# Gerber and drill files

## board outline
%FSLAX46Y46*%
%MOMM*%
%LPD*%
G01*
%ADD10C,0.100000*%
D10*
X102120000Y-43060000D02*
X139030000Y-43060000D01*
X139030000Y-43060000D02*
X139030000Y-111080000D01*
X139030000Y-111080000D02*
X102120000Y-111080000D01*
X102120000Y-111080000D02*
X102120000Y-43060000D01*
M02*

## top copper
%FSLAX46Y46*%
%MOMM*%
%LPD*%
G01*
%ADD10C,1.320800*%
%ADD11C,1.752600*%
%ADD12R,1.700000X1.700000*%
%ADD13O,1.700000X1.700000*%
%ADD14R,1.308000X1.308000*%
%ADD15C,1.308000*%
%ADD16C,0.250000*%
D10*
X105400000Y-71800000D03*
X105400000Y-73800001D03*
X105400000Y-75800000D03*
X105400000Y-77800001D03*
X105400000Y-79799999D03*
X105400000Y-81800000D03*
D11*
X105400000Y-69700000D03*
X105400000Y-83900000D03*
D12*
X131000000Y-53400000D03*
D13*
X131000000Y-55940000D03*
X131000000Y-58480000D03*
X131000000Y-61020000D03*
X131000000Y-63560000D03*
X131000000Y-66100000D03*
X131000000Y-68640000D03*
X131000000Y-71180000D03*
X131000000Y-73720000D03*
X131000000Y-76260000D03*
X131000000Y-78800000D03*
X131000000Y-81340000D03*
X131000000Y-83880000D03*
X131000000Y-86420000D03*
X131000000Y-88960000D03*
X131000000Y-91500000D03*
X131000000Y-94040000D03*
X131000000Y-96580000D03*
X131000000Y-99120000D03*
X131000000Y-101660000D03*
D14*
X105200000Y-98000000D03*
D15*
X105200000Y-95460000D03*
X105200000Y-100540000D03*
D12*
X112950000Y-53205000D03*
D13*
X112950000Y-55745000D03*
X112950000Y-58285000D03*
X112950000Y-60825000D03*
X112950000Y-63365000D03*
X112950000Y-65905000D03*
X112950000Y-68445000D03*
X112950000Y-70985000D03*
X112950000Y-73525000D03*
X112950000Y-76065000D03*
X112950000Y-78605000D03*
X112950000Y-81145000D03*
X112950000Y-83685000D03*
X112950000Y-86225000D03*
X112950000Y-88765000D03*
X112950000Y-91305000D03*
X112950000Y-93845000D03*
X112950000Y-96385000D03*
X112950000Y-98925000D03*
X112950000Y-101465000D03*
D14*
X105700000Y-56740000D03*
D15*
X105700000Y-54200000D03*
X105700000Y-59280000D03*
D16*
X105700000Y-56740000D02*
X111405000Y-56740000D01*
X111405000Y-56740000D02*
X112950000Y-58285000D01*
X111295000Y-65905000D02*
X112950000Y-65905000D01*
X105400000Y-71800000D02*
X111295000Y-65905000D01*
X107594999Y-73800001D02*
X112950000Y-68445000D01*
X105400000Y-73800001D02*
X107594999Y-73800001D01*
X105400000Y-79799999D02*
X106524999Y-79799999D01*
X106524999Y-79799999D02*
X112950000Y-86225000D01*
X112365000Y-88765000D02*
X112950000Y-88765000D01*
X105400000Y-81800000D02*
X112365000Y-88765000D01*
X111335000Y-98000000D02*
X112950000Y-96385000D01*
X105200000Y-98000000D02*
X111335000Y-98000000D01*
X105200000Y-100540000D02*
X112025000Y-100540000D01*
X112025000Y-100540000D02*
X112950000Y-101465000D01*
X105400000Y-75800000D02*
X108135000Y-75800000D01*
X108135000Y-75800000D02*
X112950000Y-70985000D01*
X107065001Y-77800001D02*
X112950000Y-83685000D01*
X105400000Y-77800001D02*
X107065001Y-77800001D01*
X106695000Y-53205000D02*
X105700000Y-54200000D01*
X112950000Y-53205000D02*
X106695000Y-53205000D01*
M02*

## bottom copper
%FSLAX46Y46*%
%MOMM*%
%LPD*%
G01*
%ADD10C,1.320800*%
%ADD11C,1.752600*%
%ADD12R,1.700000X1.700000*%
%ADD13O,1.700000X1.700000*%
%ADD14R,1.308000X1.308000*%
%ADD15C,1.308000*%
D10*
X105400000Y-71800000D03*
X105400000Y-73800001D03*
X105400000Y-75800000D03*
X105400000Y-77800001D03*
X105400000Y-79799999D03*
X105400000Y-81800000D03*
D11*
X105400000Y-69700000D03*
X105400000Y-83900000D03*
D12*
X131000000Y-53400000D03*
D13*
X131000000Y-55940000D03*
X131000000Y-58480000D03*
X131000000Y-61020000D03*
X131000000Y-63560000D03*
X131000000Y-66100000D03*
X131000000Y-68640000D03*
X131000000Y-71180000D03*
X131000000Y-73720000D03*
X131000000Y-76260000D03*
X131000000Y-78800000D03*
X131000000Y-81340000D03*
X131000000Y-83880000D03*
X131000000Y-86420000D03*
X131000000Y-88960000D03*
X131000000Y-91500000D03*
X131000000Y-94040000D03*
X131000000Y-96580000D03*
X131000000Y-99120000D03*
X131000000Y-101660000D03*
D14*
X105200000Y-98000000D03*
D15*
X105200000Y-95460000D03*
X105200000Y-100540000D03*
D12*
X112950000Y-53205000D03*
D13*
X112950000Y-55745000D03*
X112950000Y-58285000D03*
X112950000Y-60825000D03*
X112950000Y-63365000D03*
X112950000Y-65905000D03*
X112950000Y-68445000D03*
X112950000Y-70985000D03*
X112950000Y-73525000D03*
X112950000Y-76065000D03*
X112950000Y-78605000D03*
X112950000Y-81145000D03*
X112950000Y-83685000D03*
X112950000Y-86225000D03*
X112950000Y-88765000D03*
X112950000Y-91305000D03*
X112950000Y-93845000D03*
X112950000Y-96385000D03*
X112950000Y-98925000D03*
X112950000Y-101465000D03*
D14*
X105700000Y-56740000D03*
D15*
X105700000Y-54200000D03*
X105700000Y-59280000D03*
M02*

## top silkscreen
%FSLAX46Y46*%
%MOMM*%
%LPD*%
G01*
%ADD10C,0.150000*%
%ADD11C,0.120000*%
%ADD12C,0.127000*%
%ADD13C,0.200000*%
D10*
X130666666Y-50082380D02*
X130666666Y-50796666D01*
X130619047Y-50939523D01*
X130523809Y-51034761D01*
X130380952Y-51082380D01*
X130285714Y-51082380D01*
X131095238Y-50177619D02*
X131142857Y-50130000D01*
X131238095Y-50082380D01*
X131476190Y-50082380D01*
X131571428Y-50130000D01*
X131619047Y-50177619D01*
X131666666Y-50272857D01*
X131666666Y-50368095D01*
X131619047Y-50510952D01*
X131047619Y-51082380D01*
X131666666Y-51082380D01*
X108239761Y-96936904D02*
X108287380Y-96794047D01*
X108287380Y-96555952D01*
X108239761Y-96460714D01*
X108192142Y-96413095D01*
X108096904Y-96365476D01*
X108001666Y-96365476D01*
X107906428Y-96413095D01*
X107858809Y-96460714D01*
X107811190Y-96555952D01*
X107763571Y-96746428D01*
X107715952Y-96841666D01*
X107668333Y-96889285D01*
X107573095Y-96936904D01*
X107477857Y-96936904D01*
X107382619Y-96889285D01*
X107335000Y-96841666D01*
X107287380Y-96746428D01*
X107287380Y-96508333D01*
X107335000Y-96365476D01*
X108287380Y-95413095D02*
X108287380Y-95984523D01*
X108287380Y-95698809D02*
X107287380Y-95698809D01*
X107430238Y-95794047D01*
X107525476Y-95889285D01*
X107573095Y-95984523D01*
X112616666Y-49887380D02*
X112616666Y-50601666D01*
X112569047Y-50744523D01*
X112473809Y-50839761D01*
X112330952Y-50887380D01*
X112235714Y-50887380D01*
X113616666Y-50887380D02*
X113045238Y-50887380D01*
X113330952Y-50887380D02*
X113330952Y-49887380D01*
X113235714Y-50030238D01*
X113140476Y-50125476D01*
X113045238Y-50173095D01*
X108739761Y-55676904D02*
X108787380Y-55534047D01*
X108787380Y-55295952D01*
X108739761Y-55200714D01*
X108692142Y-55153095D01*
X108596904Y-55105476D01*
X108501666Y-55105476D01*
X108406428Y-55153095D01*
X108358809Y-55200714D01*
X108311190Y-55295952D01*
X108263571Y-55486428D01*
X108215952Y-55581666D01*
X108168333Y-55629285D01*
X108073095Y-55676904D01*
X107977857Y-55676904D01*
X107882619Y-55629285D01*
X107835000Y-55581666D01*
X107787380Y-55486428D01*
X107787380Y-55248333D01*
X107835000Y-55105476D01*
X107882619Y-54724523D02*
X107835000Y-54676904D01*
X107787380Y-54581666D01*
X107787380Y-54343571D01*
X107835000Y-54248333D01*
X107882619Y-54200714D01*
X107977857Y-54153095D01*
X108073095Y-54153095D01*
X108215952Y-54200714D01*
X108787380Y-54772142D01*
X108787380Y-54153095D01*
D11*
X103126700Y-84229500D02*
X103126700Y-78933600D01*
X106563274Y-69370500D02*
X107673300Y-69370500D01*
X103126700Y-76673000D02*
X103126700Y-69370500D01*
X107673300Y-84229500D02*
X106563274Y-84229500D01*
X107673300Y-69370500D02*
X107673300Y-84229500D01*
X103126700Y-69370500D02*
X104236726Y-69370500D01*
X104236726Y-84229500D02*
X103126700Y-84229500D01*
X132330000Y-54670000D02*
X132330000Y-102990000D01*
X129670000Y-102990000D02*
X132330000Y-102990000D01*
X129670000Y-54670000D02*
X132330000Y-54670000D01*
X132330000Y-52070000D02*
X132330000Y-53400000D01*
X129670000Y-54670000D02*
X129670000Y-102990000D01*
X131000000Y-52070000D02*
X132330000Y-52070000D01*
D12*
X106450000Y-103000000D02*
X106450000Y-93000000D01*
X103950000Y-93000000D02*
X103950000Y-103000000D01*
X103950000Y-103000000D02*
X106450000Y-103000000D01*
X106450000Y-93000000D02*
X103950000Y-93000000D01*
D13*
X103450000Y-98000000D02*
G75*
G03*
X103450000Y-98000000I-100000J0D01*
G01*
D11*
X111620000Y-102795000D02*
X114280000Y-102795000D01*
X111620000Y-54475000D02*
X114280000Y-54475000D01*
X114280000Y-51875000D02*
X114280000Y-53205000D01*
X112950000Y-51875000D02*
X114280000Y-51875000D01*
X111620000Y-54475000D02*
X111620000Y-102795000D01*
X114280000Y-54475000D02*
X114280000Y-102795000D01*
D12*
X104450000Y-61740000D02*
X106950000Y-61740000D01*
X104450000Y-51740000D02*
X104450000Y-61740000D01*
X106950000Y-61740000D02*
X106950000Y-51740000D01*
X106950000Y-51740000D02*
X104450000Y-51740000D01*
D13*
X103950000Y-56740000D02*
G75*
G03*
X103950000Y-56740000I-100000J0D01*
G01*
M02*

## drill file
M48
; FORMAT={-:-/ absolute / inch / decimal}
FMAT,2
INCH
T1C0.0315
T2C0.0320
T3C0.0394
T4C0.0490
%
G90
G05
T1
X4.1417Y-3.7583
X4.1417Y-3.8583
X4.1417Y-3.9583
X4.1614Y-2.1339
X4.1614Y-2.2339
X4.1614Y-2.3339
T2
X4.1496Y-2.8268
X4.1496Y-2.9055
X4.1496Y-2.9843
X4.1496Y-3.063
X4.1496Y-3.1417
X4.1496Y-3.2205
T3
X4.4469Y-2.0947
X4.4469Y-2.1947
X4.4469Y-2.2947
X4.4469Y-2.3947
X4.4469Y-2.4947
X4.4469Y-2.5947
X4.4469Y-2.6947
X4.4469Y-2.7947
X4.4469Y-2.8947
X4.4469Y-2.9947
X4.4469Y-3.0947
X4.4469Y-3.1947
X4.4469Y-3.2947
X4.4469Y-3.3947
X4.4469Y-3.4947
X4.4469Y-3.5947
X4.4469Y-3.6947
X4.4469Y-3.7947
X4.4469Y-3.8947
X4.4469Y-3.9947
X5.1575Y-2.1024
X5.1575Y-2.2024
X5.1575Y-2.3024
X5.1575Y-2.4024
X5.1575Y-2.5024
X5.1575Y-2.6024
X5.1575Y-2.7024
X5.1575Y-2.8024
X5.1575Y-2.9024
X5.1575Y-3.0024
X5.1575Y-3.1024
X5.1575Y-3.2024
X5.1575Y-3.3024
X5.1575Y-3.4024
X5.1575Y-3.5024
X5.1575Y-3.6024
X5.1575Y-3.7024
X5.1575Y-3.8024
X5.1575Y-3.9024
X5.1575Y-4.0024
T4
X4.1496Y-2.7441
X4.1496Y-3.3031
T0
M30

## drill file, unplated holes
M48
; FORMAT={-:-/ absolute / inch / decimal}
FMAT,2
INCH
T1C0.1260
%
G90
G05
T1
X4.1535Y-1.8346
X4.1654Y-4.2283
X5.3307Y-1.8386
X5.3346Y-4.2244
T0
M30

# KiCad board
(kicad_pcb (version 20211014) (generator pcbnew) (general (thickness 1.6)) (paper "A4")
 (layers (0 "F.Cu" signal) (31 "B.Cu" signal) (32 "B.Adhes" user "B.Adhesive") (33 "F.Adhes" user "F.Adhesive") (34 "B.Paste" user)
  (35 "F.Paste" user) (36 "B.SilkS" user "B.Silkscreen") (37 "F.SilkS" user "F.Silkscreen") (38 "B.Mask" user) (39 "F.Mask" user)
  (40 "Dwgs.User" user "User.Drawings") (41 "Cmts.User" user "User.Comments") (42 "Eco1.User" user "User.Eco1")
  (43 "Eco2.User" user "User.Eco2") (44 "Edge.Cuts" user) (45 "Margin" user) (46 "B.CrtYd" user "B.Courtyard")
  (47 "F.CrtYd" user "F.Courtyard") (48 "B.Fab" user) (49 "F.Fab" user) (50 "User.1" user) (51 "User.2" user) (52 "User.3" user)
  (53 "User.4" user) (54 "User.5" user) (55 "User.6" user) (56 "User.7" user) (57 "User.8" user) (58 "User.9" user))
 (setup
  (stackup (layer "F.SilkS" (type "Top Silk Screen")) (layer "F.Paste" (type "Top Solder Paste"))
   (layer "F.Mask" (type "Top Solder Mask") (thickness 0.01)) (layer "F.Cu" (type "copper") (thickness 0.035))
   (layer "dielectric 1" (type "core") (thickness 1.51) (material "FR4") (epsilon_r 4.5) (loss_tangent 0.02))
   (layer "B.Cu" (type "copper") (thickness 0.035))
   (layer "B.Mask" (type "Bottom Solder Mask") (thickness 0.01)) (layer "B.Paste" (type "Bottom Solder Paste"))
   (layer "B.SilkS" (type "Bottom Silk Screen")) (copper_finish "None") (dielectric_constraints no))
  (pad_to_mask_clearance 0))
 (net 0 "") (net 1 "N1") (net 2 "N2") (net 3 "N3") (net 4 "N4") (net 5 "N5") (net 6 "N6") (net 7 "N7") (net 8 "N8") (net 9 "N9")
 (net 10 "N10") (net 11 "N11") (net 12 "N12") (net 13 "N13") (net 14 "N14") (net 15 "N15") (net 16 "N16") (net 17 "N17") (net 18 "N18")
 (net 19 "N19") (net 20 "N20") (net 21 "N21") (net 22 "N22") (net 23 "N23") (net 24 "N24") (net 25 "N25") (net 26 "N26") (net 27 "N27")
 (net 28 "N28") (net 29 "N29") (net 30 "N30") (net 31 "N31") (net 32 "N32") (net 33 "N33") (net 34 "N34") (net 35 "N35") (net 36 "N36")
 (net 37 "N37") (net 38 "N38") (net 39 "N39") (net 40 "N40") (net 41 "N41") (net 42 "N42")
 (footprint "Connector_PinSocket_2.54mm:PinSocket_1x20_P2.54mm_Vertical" (layer "F.Cu") (at 131 53.4)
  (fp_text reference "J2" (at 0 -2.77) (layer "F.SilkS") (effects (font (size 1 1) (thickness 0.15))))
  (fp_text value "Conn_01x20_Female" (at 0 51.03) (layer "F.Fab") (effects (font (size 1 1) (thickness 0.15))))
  (fp_line (start 1.33 1.27) (end 1.33 49.59) (layer "F.SilkS") (width 0.12))
  (fp_line (start -1.33 49.59) (end 1.33 49.59) (layer "F.SilkS") (width 0.12))
  (fp_line (start -1.33 1.27) (end 1.33 1.27) (layer "F.SilkS") (width 0.12))
  (fp_line (start 1.33 -1.33) (end 1.33 0) (layer "F.SilkS") (width 0.12))
  (fp_line (start -1.33 1.27) (end -1.33 49.59) (layer "F.SilkS") (width 0.12))
  (fp_line (start 0 -1.33) (end 1.33 -1.33) (layer "F.SilkS") (width 0.12))
  (pad "1" thru_hole rect locked (at 0 0) (size 1.7 1.7) (drill 1) (layers *.Cu *.Mask) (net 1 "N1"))
  (pad "2" thru_hole oval locked (at 0 2.54) (size 1.7 1.7) (drill 1) (layers *.Cu *.Mask) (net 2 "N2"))
  (pad "3" thru_hole oval locked (at 0 5.08) (size 1.7 1.7) (drill 1) (layers *.Cu *.Mask) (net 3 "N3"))
  (pad "4" thru_hole oval locked (at 0 7.62) (size 1.7 1.7) (drill 1) (layers *.Cu *.Mask) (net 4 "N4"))
  (pad "5" thru_hole oval locked (at 0 10.16) (size 1.7 1.7) (drill 1) (layers *.Cu *.Mask) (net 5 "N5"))
  (pad "6" thru_hole oval locked (at 0 12.7) (size 1.7 1.7) (drill 1) (layers *.Cu *.Mask) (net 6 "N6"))
  (pad "7" thru_hole oval locked (at 0 15.24) (size 1.7 1.7) (drill 1) (layers *.Cu *.Mask) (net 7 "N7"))
  (pad "8" thru_hole oval locked (at 0 17.78) (size 1.7 1.7) (drill 1) (layers *.Cu *.Mask) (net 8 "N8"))
  (pad "9" thru_hole oval locked (at 0 20.32) (size 1.7 1.7) (drill 1) (layers *.Cu *.Mask) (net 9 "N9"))
  (pad "10" thru_hole oval locked (at 0 22.86) (size 1.7 1.7) (drill 1) (layers *.Cu *.Mask) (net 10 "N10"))
  (pad "11" thru_hole oval locked (at 0 25.4) (size 1.7 1.7) (drill 1) (layers *.Cu *.Mask) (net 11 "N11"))
  (pad "12" thru_hole oval locked (at 0 27.94) (size 1.7 1.7) (drill 1) (layers *.Cu *.Mask) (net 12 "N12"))
  (pad "13" thru_hole oval locked (at 0 30.48) (size 1.7 1.7) (drill 1) (layers *.Cu *.Mask) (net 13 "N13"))
  (pad "14" thru_hole oval locked (at 0 33.02) (size 1.7 1.7) (drill 1) (layers *.Cu *.Mask) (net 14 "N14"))
  (pad "15" thru_hole oval locked (at 0 35.56) (size 1.7 1.7) (drill 1) (layers *.Cu *.Mask) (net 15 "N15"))
  (pad "16" thru_hole oval locked (at 0 38.1) (size 1.7 1.7) (drill 1) (layers *.Cu *.Mask) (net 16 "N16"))
  (pad "17" thru_hole oval locked (at 0 40.64) (size 1.7 1.7) (drill 1) (layers *.Cu *.Mask) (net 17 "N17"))
  (pad "18" thru_hole oval locked (at 0 43.18) (size 1.7 1.7) (drill 1) (layers *.Cu *.Mask) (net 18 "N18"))
  (pad "19" thru_hole oval locked (at 0 45.72) (size 1.7 1.7) (drill 1) (layers *.Cu *.Mask) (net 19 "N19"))
  (pad "20" thru_hole oval locked (at 0 48.26) (size 1.7 1.7) (drill 1) (layers *.Cu *.Mask) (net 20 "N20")))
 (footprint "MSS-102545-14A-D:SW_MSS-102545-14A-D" (layer "F.Cu") (at 105.2 98 -90)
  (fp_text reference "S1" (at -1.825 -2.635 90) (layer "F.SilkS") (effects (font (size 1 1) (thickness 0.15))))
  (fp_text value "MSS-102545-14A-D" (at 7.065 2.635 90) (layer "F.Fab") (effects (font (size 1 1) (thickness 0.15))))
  (fp_line (start 5 -1.25) (end -5 -1.25) (layer "F.SilkS") (width 0.127))
  (fp_line (start -5 1.25) (end 5 1.25) (layer "F.SilkS") (width 0.127))
  (fp_line (start 5 1.25) (end 5 -1.25) (layer "F.SilkS") (width 0.127))
  (fp_line (start -5 -1.25) (end -5 1.25) (layer "F.SilkS") (width 0.127))
  (fp_circle (center 0 1.85) (end 0.1 1.85) (layer "F.SilkS") (width 0.2) (fill none))
  (pad "1" thru_hole rect locked (at 0 0 270) (size 1.308 1.308) (drill 0.8) (layers *.Cu *.Mask) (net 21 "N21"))
  (pad "2" thru_hole circle locked (at -2.54 0 270) (size 1.308 1.308) (drill 0.8) (layers *.Cu *.Mask) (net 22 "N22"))
  (pad "3" thru_hole circle locked (at 2.54 0 270) (size 1.308 1.308) (drill 0.8) (layers *.Cu *.Mask) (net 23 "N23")))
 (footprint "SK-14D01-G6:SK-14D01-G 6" (layer "F.Cu") (at 105.4 71.8 -90)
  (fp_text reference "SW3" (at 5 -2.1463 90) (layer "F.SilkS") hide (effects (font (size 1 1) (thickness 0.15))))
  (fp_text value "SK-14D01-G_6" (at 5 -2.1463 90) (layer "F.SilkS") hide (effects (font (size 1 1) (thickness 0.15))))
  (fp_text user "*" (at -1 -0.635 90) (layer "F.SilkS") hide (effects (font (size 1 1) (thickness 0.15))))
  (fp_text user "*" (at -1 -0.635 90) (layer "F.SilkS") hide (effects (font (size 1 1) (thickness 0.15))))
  (fp_line (start 12.4295 2.2733) (end 7.1336 2.2733) (layer "F.SilkS") (width 0.12))
  (fp_line (start -2.4295 -1.163274) (end -2.4295 -2.2733) (layer "F.SilkS") (width 0.12))
  (fp_line (start 4.873 2.2733) (end -2.4295 2.2733) (layer "F.SilkS") (width 0.12))
  (fp_line (start 12.4295 -2.2733) (end 12.4295 -1.163274) (layer "F.SilkS") (width 0.12))
  (fp_line (start -2.4295 -2.2733) (end 12.4295 -2.2733) (layer "F.SilkS") (width 0.12))
  (fp_line (start -2.4295 2.2733) (end -2.4295 1.163274) (layer "F.SilkS") (width 0.12))
  (fp_line (start 12.4295 1.163274) (end 12.4295 2.2733) (layer "F.SilkS") (width 0.12))
  (pad "1" thru_hole circle (at 0 0 270) (size 1.3208 1.3208) (drill 0.8128) (layers *.Cu *.Mask) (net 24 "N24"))
  (pad "2" thru_hole circle (at 2.000001 0 270) (size 1.3208 1.3208) (drill 0.8128) (layers *.Cu *.Mask) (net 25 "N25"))
  (pad "3" thru_hole circle (at 4 0 270) (size 1.3208 1.3208) (drill 0.8128) (layers *.Cu *.Mask) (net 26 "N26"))
  (pad "4" thru_hole circle (at 6.000001 0 270) (size 1.3208 1.3208) (drill 0.8128) (layers *.Cu *.Mask) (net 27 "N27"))
  (pad "5" thru_hole circle (at 7.999999 0 270) (size 1.3208 1.3208) (drill 0.8128) (layers *.Cu *.Mask) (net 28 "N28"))
  (pad "6" thru_hole circle (at 10 0 270) (size 1.3208 1.3208) (drill 0.8128) (layers *.Cu *.Mask) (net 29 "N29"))
  (pad "7" thru_hole circle (at -2.1 0 270) (size 1.7526 1.7526) (drill 1.2446) (layers *.Cu *.Mask))
  (pad "8" thru_hole circle (at 12.1 0 270) (size 1.7526 1.7526) (drill 1.2446) (layers *.Cu *.Mask)))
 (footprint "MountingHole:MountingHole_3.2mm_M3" (layer "F.Cu") (at 105.5 46.6)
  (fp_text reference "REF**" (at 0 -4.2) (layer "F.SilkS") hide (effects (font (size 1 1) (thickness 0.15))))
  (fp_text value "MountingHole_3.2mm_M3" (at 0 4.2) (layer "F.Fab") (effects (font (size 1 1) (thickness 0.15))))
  (pad "" np_thru_hole circle (at 0 0) (size 3.2 3.2) (drill 3.2) (layers *.Cu *.Mask)))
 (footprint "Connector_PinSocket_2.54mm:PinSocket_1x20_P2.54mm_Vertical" (layer "F.Cu") (at 112.95 53.205)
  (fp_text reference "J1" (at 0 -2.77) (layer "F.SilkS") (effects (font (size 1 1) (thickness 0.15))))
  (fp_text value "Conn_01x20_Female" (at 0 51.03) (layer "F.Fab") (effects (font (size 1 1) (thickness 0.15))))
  (fp_line (start -1.33 49.59) (end 1.33 49.59) (layer "F.SilkS") (width 0.12))
  (fp_line (start -1.33 1.27) (end 1.33 1.27) (layer "F.SilkS") (width 0.12))
  (fp_line (start 1.33 -1.33) (end 1.33 0) (layer "F.SilkS") (width 0.12))
  (fp_line (start 0 -1.33) (end 1.33 -1.33) (layer "F.SilkS") (width 0.12))
  (fp_line (start -1.33 1.27) (end -1.33 49.59) (layer "F.SilkS") (width 0.12))
  (fp_line (start 1.33 1.27) (end 1.33 49.59) (layer "F.SilkS") (width 0.12))
  (pad "1" thru_hole rect locked (at 0 0) (size 1.7 1.7) (drill 1) (layers *.Cu *.Mask) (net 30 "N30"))
  (pad "2" thru_hole oval locked (at 0 2.54) (size 1.7 1.7) (drill 1) (layers *.Cu *.Mask) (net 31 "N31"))
  (pad "3" thru_hole oval locked (at 0 5.08) (size 1.7 1.7) (drill 1) (layers *.Cu *.Mask) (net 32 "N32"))
  (pad "4" thru_hole oval locked (at 0 7.62) (size 1.7 1.7) (drill 1) (layers *.Cu *.Mask) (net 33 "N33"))
  (pad "5" thru_hole oval locked (at 0 10.16) (size 1.7 1.7) (drill 1) (layers *.Cu *.Mask) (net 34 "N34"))
  (pad "6" thru_hole oval locked (at 0 12.7) (size 1.7 1.7) (drill 1) (layers *.Cu *.Mask) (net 24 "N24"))
  (pad "7" thru_hole oval locked (at 0 15.24) (size 1.7 1.7) (drill 1) (layers *.Cu *.Mask) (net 25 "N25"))
  (pad "8" thru_hole oval locked (at 0 17.78) (size 1.7 1.7) (drill 1) (layers *.Cu *.Mask) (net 26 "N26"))
  (pad "9" thru_hole oval locked (at 0 20.32) (size 1.7 1.7) (drill 1) (layers *.Cu *.Mask) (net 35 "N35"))
  (pad "10" thru_hole oval locked (at 0 22.86) (size 1.7 1.7) (drill 1) (layers *.Cu *.Mask) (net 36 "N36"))
  (pad "11" thru_hole oval locked (at 0 25.4) (size 1.7 1.7) (drill 1) (layers *.Cu *.Mask) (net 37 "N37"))
  (pad "12" thru_hole oval locked (at 0 27.94) (size 1.7 1.7) (drill 1) (layers *.Cu *.Mask) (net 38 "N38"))
  (pad "13" thru_hole oval locked (at 0 30.48) (size 1.7 1.7) (drill 1) (layers *.Cu *.Mask) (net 27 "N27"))
  (pad "14" thru_hole oval locked (at 0 33.02) (size 1.7 1.7) (drill 1) (layers *.Cu *.Mask) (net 28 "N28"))
  (pad "15" thru_hole oval locked (at 0 35.56) (size 1.7 1.7) (drill 1) (layers *.Cu *.Mask) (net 29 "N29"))
  (pad "16" thru_hole oval locked (at 0 38.1) (size 1.7 1.7) (drill 1) (layers *.Cu *.Mask) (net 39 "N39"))
  (pad "17" thru_hole oval locked (at 0 40.64) (size 1.7 1.7) (drill 1) (layers *.Cu *.Mask) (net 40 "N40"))
  (pad "18" thru_hole oval locked (at 0 43.18) (size 1.7 1.7) (drill 1) (layers *.Cu *.Mask) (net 21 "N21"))
  (pad "19" thru_hole oval locked (at 0 45.72) (size 1.7 1.7) (drill 1) (layers *.Cu *.Mask) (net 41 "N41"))
  (pad "20" thru_hole oval locked (at 0 48.26) (size 1.7 1.7) (drill 1) (layers *.Cu *.Mask) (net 23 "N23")))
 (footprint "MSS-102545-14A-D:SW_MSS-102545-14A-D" (layer "F.Cu") (at 105.7 56.74 -90)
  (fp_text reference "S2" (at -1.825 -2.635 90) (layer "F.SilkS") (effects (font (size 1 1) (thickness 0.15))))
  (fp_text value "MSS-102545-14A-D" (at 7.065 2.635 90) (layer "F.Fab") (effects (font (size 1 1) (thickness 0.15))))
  (fp_line (start 5 1.25) (end 5 -1.25) (layer "F.SilkS") (width 0.127))
  (fp_line (start -5 1.25) (end 5 1.25) (layer "F.SilkS") (width 0.127))
  (fp_line (start 5 -1.25) (end -5 -1.25) (layer "F.SilkS") (width 0.127))
  (fp_line (start -5 -1.25) (end -5 1.25) (layer "F.SilkS") (width 0.127))
  (fp_circle (center 0 1.85) (end 0.1 1.85) (layer "F.SilkS") (width 0.2) (fill none))
  (pad "1" thru_hole rect locked (at 0 0 270) (size 1.308 1.308) (drill 0.8) (layers *.Cu *.Mask) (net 32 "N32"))
  (pad "2" thru_hole circle locked (at -2.54 0 270) (size 1.308 1.308) (drill 0.8) (layers *.Cu *.Mask) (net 30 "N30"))
  (pad "3" thru_hole circle locked (at 2.54 0 270) (size 1.308 1.308) (drill 0.8) (layers *.Cu *.Mask) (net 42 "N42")))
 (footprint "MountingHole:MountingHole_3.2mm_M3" (layer "F.Cu") (at 135.4 46.7)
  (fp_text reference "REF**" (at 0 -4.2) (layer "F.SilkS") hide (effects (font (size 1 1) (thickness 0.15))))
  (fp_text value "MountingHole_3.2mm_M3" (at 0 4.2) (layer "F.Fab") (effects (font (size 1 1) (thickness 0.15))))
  (pad "" np_thru_hole circle (at 0 0) (size 3.2 3.2) (drill 3.2) (layers *.Cu *.Mask)))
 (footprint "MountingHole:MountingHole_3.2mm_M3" (layer "F.Cu") (at 135.5 107.3)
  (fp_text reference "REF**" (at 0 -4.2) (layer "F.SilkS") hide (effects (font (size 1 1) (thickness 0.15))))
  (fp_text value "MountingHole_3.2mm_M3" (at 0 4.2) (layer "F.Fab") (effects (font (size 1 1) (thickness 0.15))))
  (pad "" np_thru_hole circle (at 0 0) (size 3.2 3.2) (drill 3.2) (layers *.Cu *.Mask)))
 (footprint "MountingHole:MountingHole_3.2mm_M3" (layer "F.Cu") (at 105.8 107.4)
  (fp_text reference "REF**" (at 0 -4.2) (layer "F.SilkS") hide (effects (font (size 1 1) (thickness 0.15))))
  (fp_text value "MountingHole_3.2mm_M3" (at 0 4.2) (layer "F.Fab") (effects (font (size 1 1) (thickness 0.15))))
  (pad "" np_thru_hole circle (at 0 0) (size 3.2 3.2) (drill 3.2) (layers *.Cu *.Mask)))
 (gr_rect (start 102.12 43.06) (end 139.03 111.08) (layer "Edge.Cuts") (width 0.1) (fill none))
 (segment (start 105.7 56.74) (end 111.405 56.74) (width 0.25) (layer "F.Cu") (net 32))
 (segment (start 111.405 56.74) (end 112.95 58.285) (width 0.25) (layer "F.Cu") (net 32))
 (segment (start 111.295 65.905) (end 112.95 65.905) (width 0.25) (layer "F.Cu") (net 24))
 (segment (start 105.4 71.8) (end 111.295 65.905) (width 0.25) (layer "F.Cu") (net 24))
 (segment (start 107.594999 73.800001) (end 112.95 68.445) (width 0.25) (layer "F.Cu") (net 25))
 (segment (start 105.4 73.800001) (end 107.594999 73.800001) (width 0.25) (layer "F.Cu") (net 25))
 (segment (start 105.4 79.799999) (end 106.524999 79.799999) (width 0.25) (layer "F.Cu") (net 28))
 (segment (start 106.524999 79.799999) (end 112.95 86.225) (width 0.25) (layer "F.Cu") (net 28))
 (segment (start 112.365 88.765) (end 112.95 88.765) (width 0.25) (layer "F.Cu") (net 29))
 (segment (start 105.4 81.8) (end 112.365 88.765) (width 0.25) (layer "F.Cu") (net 29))
 (segment (start 111.335 98) (end 112.95 96.385) (width 0.25) (layer "F.Cu") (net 21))
 (segment (start 105.2 98) (end 111.335 98) (width 0.25) (layer "F.Cu") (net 21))
 (segment (start 105.2 100.54) (end 112.025 100.54) (width 0.25) (layer "F.Cu") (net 23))
 (segment (start 112.025 100.54) (end 112.95 101.465) (width 0.25) (layer "F.Cu") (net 23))
 (segment (start 105.4 75.8) (end 108.135 75.8) (width 0.25) (layer "F.Cu") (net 26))
 (segment (start 108.135 75.8) (end 112.95 70.985) (width 0.25) (layer "F.Cu") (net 26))
 (segment (start 107.065001 77.800001) (end 112.95 83.685) (width 0.25) (layer "F.Cu") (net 27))
 (segment (start 105.4 77.800001) (end 107.065001 77.800001) (width 0.25) (layer "F.Cu") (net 27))
 (segment (start 106.695 53.205) (end 105.7 54.2) (width 0.25) (layer "F.Cu") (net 30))
 (segment (start 112.95 53.205) (end 106.695 53.205) (width 0.25) (layer "F.Cu") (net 30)))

